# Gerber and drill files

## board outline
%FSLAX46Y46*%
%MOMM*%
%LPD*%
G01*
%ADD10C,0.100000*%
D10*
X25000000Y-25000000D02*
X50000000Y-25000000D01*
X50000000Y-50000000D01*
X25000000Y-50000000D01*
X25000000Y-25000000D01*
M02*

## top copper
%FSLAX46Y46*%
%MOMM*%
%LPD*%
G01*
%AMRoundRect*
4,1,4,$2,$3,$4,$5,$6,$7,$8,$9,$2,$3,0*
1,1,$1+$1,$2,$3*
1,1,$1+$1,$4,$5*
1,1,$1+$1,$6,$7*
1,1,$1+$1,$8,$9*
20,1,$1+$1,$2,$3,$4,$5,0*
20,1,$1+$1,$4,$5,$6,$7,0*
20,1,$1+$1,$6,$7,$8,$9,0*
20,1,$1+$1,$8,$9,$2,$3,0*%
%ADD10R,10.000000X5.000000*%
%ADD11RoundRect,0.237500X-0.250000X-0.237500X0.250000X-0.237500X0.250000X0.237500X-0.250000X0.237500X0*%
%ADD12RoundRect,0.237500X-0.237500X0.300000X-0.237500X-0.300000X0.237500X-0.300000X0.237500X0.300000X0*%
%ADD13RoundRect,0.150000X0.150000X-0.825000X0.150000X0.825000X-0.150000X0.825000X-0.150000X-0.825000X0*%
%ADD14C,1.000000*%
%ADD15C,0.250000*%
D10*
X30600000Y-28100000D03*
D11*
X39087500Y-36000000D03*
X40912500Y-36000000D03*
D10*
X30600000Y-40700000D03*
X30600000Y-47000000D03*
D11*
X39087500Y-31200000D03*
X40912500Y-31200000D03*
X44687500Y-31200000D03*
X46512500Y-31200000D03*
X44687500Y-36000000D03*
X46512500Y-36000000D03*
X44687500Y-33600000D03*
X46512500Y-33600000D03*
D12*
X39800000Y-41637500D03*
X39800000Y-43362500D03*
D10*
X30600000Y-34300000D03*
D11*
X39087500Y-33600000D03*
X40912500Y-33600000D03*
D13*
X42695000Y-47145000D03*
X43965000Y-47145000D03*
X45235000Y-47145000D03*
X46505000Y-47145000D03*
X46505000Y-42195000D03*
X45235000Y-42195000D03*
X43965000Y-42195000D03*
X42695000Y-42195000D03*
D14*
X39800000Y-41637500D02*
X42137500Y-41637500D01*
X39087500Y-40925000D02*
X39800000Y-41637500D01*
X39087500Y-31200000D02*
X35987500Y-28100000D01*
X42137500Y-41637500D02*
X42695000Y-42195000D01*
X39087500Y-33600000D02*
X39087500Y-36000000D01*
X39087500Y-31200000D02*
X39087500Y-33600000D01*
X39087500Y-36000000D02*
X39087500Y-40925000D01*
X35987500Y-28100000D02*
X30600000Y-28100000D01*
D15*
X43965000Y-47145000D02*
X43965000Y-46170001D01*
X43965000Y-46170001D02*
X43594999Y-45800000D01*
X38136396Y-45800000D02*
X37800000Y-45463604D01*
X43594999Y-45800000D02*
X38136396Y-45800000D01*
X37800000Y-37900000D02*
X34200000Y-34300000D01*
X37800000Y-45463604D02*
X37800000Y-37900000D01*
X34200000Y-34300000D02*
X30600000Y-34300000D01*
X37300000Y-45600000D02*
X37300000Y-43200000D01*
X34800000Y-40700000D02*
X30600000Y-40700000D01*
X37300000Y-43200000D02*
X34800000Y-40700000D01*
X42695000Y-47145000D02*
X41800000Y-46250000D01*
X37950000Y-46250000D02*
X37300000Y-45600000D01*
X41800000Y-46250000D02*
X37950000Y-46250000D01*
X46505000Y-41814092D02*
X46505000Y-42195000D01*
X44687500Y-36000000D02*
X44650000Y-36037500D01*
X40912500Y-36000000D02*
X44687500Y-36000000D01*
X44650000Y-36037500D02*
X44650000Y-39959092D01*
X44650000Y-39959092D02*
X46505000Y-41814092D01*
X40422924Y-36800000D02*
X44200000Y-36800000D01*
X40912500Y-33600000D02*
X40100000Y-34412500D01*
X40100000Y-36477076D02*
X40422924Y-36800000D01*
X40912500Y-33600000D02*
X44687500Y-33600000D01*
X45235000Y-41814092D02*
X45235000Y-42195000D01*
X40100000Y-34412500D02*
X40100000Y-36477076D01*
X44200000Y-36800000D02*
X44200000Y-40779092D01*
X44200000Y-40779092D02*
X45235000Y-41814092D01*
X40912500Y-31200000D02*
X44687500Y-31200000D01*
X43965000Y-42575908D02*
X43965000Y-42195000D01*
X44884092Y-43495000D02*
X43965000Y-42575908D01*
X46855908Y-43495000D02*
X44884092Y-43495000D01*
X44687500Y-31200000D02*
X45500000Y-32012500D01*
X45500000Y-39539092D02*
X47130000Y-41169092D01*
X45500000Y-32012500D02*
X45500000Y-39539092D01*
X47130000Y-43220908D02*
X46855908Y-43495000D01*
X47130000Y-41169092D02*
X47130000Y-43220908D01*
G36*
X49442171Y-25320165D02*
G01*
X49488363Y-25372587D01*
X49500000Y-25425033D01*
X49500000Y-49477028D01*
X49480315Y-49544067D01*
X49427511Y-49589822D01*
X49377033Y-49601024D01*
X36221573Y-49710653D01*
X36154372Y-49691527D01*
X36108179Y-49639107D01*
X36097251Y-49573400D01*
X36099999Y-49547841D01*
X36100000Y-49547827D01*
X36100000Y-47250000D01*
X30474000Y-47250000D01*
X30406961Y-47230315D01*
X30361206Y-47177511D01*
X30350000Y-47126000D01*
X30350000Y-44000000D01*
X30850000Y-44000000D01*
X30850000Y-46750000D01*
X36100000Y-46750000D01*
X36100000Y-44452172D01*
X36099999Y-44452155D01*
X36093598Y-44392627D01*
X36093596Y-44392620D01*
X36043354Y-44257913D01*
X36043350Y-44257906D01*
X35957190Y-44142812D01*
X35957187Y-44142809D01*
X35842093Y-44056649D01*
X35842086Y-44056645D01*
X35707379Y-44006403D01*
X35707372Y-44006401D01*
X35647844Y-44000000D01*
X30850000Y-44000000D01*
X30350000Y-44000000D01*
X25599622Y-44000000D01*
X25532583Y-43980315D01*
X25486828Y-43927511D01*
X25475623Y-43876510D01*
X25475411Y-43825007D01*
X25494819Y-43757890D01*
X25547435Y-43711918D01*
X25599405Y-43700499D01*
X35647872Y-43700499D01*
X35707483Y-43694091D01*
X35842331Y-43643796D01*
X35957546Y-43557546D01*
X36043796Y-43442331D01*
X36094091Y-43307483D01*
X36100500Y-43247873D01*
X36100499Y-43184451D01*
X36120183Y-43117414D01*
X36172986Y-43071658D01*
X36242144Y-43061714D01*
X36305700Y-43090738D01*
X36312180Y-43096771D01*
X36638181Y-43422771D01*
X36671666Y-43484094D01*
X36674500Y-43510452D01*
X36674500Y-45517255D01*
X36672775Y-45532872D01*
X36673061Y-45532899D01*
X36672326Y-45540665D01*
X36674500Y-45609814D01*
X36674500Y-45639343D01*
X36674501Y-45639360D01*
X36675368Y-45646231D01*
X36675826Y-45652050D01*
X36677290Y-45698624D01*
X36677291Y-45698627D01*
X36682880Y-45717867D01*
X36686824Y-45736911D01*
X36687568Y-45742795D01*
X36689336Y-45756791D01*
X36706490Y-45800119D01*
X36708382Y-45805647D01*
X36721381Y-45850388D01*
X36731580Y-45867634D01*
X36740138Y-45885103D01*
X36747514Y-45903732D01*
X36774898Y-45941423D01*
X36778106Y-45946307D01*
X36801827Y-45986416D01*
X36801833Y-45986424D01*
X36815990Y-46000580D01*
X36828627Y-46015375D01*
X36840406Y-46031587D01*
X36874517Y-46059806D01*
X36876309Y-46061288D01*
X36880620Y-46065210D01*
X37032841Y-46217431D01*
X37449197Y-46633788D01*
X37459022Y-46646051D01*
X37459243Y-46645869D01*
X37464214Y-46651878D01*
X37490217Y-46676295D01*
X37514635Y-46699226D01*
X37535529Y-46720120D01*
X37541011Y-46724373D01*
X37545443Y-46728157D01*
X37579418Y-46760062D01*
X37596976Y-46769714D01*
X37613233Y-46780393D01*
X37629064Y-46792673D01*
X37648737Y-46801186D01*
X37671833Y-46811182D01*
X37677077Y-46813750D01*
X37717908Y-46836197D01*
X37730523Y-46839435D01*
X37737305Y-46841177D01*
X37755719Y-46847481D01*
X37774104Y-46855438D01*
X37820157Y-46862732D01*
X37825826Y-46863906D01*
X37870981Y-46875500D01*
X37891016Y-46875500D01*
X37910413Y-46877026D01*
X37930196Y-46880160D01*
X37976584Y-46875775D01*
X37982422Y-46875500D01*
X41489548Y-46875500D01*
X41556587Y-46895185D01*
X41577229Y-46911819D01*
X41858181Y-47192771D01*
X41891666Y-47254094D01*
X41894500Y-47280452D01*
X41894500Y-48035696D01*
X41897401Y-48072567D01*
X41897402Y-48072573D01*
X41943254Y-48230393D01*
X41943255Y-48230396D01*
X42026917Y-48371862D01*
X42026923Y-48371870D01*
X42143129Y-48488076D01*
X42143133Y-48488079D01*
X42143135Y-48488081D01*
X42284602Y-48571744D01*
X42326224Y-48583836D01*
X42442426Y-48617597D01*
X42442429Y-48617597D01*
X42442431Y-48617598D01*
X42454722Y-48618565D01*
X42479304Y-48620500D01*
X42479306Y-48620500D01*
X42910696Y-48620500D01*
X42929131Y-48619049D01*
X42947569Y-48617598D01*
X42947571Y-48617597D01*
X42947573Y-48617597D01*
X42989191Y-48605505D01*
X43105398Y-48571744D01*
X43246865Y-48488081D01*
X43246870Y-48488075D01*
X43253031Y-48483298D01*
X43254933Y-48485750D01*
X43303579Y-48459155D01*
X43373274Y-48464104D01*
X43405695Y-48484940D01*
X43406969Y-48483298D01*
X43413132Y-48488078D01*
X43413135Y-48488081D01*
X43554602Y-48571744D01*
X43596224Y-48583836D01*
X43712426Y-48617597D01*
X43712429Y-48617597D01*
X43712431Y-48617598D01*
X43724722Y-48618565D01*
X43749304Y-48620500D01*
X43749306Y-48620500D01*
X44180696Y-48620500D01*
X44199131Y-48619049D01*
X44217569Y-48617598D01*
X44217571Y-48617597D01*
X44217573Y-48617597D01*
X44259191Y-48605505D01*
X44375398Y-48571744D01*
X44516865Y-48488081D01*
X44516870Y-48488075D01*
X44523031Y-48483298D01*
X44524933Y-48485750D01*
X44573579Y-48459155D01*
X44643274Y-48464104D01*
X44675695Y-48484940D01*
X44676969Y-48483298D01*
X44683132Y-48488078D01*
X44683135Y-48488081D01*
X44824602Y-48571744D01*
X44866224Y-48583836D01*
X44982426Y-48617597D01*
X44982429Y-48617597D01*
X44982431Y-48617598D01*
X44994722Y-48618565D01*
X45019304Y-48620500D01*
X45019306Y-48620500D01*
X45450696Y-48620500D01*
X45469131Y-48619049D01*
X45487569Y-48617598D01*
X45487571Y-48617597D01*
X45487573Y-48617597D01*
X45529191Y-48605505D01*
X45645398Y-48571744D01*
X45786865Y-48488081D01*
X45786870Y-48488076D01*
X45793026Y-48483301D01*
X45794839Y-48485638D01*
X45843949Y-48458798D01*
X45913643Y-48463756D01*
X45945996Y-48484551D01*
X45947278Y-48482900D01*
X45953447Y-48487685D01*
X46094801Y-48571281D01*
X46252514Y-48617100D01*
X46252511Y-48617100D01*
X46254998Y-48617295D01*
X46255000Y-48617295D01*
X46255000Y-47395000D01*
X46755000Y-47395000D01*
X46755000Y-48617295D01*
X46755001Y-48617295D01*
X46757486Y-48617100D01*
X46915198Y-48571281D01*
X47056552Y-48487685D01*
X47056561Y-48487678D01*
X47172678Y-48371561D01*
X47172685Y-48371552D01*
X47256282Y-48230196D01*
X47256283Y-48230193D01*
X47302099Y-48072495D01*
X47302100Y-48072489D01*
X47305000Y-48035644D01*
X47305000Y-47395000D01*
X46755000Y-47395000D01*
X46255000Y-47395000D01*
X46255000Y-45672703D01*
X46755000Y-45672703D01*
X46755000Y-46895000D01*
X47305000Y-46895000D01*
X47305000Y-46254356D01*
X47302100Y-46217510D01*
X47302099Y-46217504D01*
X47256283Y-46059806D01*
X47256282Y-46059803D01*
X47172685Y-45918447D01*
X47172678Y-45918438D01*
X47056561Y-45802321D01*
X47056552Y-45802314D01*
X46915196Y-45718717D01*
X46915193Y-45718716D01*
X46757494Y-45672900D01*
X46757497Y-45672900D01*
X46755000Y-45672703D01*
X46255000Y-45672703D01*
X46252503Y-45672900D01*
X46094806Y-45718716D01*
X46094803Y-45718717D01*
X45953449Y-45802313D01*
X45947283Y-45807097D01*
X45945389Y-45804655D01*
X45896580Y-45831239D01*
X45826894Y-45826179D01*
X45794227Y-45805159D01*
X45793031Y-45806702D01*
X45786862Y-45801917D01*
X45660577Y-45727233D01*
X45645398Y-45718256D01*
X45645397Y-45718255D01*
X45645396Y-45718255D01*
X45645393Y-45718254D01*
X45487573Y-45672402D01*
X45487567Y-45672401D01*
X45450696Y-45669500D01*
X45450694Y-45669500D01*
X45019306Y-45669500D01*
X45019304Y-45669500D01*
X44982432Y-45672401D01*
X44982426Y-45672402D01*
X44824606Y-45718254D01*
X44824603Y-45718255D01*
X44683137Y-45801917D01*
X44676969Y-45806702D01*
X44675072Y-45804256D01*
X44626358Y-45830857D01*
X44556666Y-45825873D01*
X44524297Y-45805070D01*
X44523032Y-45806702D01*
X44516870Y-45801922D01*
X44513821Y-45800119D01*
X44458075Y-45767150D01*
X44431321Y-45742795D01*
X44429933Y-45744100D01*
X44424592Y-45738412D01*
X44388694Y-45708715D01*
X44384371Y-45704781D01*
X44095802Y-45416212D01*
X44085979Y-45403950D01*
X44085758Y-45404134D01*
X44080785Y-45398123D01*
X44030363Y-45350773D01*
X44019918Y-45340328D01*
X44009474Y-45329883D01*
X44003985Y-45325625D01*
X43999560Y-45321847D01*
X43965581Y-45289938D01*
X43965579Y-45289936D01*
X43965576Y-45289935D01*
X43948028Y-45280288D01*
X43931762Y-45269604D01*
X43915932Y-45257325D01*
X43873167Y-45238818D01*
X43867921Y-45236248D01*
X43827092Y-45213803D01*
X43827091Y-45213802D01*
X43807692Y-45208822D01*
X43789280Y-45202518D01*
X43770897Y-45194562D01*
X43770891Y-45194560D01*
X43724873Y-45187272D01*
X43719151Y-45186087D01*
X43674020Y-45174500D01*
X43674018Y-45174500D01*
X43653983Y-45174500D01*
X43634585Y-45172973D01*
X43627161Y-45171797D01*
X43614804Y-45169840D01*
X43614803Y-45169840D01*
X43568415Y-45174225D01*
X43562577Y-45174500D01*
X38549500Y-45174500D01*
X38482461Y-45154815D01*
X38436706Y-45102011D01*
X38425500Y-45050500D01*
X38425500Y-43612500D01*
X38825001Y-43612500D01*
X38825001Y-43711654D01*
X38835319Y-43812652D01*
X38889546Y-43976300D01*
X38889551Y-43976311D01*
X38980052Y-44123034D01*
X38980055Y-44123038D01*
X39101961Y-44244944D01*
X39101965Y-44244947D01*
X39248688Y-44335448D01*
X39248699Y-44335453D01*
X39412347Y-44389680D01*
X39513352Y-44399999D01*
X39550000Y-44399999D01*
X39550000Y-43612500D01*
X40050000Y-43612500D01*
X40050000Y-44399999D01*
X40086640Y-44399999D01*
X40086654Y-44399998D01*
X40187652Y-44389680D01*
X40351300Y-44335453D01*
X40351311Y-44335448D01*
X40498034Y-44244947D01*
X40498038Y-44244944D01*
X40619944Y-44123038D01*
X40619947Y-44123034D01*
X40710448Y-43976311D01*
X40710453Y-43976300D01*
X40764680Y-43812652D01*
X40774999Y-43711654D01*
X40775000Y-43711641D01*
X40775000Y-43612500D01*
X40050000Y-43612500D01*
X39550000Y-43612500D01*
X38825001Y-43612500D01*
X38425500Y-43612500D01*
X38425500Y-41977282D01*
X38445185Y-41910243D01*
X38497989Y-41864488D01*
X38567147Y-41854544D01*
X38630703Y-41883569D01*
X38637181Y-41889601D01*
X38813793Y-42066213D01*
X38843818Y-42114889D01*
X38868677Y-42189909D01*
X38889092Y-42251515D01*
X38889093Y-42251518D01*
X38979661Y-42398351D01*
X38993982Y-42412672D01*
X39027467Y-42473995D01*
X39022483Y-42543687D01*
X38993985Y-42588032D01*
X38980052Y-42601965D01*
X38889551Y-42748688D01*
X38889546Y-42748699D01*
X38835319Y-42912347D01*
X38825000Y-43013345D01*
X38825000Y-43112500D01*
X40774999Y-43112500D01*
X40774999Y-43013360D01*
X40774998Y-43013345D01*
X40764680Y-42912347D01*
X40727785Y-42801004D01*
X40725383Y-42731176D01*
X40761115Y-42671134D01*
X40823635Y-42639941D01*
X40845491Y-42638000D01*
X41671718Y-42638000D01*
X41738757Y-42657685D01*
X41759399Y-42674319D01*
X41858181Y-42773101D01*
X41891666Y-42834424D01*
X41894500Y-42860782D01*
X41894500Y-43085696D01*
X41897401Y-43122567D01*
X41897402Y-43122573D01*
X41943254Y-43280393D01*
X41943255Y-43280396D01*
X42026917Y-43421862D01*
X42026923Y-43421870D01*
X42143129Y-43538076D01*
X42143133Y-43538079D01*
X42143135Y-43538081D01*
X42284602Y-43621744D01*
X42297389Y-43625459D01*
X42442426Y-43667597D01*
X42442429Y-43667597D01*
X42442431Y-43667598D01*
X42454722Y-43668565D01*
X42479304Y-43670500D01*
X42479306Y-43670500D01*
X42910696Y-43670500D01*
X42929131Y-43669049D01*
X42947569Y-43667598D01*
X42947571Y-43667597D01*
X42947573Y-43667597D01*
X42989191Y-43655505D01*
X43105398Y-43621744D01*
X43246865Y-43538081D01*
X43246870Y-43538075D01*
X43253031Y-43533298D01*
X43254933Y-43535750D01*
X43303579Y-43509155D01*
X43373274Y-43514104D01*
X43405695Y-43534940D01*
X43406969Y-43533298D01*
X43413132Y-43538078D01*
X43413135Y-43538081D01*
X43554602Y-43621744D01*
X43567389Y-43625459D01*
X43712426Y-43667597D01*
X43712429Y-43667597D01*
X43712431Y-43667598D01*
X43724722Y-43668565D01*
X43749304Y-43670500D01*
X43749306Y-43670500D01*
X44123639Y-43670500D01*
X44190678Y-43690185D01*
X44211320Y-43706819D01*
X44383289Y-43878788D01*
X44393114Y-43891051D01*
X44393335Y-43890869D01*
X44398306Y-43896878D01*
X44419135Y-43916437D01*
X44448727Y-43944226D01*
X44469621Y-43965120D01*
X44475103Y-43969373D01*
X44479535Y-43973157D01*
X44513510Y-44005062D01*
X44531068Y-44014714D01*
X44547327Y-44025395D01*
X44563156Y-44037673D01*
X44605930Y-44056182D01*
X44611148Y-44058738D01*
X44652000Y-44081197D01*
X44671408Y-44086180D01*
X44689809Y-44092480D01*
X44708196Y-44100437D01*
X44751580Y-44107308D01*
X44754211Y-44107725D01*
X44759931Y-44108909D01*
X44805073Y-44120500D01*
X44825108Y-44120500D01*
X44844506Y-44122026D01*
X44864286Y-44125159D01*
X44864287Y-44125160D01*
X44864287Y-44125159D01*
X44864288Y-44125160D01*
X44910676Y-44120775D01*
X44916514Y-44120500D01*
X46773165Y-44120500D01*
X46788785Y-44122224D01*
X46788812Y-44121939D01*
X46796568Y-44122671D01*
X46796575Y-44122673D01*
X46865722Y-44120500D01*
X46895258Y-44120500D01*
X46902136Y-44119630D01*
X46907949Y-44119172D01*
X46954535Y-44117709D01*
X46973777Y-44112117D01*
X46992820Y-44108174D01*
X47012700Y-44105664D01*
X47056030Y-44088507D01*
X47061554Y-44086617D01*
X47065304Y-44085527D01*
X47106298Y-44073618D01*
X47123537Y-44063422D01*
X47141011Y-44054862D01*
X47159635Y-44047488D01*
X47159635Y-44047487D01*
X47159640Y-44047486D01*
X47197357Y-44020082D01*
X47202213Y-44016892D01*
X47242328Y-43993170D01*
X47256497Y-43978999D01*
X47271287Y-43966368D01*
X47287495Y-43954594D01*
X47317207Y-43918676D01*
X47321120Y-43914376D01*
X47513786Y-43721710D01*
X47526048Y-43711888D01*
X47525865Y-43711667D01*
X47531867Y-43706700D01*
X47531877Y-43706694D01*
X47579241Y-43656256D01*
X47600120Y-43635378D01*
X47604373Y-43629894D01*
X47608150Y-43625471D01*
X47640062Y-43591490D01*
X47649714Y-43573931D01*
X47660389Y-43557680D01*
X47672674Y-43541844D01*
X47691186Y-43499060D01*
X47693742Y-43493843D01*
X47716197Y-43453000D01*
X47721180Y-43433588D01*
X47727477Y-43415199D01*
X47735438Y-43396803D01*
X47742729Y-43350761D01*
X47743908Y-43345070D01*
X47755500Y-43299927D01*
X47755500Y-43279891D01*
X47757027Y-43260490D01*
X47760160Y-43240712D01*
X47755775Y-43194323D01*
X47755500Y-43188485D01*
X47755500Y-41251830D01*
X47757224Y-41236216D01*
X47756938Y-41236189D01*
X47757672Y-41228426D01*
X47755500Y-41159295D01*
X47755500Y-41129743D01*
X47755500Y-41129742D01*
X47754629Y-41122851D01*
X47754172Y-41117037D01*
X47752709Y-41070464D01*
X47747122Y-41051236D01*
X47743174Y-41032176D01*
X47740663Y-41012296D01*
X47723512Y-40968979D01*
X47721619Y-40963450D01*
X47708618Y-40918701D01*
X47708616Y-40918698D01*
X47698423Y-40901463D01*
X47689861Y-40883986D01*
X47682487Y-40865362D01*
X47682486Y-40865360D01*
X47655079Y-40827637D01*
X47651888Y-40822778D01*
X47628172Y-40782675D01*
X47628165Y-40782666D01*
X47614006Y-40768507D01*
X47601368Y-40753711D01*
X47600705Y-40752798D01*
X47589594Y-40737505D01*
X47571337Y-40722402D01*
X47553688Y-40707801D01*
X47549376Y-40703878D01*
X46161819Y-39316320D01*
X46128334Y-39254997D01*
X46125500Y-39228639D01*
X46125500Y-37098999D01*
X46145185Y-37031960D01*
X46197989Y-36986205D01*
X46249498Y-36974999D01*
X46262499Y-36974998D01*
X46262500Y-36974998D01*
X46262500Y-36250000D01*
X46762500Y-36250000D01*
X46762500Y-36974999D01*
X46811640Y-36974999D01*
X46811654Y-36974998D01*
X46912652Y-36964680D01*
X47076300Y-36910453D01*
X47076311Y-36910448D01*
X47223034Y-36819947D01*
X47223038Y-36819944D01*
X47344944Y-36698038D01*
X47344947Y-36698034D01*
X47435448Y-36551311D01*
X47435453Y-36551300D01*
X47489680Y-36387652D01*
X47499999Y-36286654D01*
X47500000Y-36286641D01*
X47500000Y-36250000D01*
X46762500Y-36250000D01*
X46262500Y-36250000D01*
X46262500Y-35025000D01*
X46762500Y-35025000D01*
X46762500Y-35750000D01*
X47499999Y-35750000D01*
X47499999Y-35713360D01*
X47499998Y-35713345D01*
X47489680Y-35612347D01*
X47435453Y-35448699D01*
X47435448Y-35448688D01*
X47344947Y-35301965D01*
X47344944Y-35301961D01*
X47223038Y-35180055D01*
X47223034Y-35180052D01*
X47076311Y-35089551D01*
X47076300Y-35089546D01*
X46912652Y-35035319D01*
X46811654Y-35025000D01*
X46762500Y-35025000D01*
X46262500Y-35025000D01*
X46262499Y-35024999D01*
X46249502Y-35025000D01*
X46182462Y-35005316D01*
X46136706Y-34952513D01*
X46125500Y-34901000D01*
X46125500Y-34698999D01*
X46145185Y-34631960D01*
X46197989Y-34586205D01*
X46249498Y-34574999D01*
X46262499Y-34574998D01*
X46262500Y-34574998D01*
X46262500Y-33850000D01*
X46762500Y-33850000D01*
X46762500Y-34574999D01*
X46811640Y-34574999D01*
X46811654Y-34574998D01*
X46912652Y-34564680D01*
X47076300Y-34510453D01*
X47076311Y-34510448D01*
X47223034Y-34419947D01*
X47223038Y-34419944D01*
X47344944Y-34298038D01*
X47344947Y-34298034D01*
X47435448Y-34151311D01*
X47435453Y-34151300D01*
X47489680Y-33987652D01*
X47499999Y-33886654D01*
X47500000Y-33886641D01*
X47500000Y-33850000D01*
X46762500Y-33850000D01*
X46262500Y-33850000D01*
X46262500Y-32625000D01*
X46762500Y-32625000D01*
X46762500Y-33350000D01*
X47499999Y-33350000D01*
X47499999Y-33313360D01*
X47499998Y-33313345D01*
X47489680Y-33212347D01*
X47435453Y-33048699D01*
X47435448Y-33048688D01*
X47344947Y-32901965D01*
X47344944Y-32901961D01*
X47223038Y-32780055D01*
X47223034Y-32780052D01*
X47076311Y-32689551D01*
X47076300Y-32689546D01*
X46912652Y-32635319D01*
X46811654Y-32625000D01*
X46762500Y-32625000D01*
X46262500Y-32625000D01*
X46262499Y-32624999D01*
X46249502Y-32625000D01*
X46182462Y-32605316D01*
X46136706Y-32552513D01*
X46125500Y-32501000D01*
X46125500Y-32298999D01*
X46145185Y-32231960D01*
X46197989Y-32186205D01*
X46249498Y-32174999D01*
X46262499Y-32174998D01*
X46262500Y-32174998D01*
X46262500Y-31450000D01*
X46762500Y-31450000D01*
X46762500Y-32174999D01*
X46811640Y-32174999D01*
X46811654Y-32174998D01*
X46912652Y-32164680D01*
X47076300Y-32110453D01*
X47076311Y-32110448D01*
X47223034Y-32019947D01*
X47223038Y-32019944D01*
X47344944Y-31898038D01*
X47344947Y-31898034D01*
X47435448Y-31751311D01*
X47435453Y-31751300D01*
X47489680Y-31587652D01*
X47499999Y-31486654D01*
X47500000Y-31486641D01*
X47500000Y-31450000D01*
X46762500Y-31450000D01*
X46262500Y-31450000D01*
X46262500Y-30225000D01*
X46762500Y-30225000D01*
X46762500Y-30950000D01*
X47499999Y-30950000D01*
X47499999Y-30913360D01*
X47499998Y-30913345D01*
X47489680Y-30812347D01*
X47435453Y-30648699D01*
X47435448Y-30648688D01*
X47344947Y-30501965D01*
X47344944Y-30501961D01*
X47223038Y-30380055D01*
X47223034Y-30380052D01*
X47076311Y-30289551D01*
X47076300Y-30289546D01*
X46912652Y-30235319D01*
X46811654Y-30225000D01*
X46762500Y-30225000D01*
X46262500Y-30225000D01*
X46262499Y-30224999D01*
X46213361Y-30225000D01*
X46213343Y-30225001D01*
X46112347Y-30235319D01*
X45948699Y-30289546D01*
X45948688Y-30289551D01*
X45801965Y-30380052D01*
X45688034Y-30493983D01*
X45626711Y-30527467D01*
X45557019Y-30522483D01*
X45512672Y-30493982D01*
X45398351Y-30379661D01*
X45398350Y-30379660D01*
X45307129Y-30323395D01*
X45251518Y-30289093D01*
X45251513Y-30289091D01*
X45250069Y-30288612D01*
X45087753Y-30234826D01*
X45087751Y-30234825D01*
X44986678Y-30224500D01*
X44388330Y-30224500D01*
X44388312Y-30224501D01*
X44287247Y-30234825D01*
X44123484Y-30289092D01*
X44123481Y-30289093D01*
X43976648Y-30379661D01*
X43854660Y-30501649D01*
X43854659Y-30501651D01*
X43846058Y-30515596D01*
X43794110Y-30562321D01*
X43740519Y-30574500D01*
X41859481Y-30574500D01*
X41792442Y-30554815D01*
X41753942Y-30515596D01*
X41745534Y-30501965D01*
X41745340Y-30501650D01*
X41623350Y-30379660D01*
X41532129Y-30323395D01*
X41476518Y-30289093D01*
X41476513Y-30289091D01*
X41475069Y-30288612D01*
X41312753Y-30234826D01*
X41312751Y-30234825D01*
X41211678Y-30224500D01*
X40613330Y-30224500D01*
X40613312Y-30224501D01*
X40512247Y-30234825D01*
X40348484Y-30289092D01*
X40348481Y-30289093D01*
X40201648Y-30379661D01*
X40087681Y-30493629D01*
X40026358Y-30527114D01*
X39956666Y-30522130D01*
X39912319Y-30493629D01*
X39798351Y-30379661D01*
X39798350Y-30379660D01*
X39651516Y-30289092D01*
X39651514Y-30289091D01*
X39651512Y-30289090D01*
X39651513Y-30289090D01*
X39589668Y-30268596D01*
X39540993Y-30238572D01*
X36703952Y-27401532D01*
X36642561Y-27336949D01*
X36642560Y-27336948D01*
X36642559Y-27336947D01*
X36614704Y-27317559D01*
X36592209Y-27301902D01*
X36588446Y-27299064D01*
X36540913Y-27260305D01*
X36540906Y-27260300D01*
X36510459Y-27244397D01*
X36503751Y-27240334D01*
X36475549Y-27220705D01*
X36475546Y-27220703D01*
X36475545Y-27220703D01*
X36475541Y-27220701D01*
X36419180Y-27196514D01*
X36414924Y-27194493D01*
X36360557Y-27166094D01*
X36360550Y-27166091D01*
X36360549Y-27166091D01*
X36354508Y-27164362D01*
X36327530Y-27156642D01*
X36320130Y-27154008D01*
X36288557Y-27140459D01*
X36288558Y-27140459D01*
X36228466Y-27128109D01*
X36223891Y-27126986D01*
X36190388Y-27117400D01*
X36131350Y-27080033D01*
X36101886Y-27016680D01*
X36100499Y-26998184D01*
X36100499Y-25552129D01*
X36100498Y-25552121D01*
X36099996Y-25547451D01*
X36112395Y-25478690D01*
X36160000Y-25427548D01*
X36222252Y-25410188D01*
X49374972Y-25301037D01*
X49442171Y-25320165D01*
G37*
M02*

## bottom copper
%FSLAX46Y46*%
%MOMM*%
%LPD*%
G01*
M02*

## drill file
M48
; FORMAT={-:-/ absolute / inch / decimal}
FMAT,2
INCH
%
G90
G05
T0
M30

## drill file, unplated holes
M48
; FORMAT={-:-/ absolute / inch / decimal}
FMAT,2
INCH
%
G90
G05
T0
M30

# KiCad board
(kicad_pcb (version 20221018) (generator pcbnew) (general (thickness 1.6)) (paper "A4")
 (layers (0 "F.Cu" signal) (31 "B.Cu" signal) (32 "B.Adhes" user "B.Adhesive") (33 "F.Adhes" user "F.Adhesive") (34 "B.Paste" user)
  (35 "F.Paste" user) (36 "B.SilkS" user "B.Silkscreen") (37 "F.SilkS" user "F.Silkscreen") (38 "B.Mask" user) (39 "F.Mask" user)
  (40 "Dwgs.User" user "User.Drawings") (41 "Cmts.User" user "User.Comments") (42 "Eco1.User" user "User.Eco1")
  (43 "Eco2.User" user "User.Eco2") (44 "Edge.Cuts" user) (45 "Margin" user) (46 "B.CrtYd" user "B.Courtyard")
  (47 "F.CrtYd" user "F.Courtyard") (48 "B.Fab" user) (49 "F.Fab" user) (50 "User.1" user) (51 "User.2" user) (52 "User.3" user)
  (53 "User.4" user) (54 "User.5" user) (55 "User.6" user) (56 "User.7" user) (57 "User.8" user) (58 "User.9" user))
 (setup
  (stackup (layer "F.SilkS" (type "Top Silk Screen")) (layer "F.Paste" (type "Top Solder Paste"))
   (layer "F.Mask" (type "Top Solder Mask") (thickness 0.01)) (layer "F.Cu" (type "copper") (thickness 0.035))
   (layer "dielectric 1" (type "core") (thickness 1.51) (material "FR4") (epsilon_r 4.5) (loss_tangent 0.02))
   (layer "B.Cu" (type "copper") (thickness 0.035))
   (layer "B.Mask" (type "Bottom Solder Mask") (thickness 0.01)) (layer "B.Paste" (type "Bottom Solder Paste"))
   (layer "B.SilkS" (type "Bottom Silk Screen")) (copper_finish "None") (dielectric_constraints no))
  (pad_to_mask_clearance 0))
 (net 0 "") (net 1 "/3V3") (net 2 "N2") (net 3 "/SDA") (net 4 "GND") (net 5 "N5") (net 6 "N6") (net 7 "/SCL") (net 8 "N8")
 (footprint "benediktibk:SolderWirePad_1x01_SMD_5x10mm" (layer "F.Cu") (at 30.6 28.1 -90)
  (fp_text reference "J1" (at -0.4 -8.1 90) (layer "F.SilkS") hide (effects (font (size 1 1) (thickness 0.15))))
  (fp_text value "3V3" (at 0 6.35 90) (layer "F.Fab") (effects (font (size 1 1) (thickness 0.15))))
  (pad "1" smd rect (at 0 0 270) (size 5 10) (layers "F.Cu" "F.Paste" "F.Mask") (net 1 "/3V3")))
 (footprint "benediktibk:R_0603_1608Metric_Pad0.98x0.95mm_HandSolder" (layer "F.Cu") (at 40 36)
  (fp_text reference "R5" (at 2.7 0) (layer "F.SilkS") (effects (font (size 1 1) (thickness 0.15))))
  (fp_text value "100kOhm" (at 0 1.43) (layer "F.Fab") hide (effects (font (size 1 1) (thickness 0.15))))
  (pad "1" smd roundrect (at -0.9125 0) (size 0.975 0.95) (layers "F.Cu" "F.Paste" "F.Mask") (roundrect_rratio 0.25) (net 1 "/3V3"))
  (pad "2" smd roundrect (at 0.9125 0) (size 0.975 0.95) (layers "F.Cu" "F.Paste" "F.Mask") (roundrect_rratio 0.25) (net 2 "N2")))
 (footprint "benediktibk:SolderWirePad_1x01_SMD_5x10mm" (layer "F.Cu") (at 30.6 40.7 -90)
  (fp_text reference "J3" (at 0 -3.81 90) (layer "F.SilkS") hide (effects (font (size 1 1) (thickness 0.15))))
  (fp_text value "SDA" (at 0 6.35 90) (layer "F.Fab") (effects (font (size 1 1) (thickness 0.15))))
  (pad "1" smd rect (at 0 0 270) (size 5 10) (layers "F.Cu" "F.Paste" "F.Mask") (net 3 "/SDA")))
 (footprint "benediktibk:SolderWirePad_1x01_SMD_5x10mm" (layer "F.Cu") (at 30.6 47 -90)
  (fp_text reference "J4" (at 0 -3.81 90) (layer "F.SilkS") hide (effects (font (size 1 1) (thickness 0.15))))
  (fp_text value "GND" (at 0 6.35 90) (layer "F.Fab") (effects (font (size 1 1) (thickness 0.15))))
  (pad "1" smd rect (at 0 0 270) (size 5 10) (layers "F.Cu" "F.Paste" "F.Mask") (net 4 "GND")))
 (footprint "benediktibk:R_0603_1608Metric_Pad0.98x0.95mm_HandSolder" (layer "F.Cu") (at 40 31.2)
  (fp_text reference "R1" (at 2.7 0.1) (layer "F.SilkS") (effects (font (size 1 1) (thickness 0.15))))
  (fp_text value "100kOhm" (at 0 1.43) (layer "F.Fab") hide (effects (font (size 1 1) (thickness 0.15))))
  (pad "1" smd roundrect (at -0.9125 0) (size 0.975 0.95) (layers "F.Cu" "F.Paste" "F.Mask") (roundrect_rratio 0.25) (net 1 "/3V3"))
  (pad "2" smd roundrect (at 0.9125 0) (size 0.975 0.95) (layers "F.Cu" "F.Paste" "F.Mask") (roundrect_rratio 0.25) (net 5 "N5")))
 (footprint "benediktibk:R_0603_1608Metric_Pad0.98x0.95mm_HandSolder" (layer "F.Cu") (at 45.6 31.2)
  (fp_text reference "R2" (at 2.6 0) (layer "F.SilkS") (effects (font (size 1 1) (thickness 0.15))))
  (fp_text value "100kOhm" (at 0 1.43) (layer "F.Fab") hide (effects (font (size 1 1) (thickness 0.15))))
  (pad "1" smd roundrect (at -0.9125 0) (size 0.975 0.95) (layers "F.Cu" "F.Paste" "F.Mask") (roundrect_rratio 0.25) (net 5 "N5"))
  (pad "2" smd roundrect (at 0.9125 0) (size 0.975 0.95) (layers "F.Cu" "F.Paste" "F.Mask") (roundrect_rratio 0.25) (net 4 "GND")))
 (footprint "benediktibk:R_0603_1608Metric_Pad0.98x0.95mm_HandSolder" (layer "F.Cu") (at 45.6 36)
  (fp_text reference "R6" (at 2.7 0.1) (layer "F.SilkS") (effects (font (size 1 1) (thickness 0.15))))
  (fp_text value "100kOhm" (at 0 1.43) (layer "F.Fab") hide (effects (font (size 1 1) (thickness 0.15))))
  (pad "1" smd roundrect (at -0.9125 0) (size 0.975 0.95) (layers "F.Cu" "F.Paste" "F.Mask") (roundrect_rratio 0.25) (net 2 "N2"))
  (pad "2" smd roundrect (at 0.9125 0) (size 0.975 0.95) (layers "F.Cu" "F.Paste" "F.Mask") (roundrect_rratio 0.25) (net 4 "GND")))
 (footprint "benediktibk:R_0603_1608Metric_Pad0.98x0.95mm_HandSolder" (layer "F.Cu") (at 45.6 33.6)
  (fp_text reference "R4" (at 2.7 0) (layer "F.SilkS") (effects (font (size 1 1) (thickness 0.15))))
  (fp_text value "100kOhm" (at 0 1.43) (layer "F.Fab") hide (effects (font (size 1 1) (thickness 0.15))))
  (pad "1" smd roundrect (at -0.9125 0) (size 0.975 0.95) (layers "F.Cu" "F.Paste" "F.Mask") (roundrect_rratio 0.25) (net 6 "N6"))
  (pad "2" smd roundrect (at 0.9125 0) (size 0.975 0.95) (layers "F.Cu" "F.Paste" "F.Mask") (roundrect_rratio 0.25) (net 4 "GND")))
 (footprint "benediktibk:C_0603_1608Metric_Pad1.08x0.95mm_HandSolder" (layer "F.Cu") (at 39.8 42.5 -90)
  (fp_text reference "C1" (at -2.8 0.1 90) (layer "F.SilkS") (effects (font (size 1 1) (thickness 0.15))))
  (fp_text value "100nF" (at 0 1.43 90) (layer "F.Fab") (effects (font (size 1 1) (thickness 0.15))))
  (pad "1" smd roundrect (at -0.8625 0 270) (size 1.075 0.95) (layers "F.Cu" "F.Paste" "F.Mask") (roundrect_rratio 0.25) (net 1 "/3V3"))
  (pad "2" smd roundrect (at 0.8625 0 270) (size 1.075 0.95) (layers "F.Cu" "F.Paste" "F.Mask") (roundrect_rratio 0.25) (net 4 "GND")))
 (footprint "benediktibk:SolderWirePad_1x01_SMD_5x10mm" (layer "F.Cu") (at 30.6 34.3 -90)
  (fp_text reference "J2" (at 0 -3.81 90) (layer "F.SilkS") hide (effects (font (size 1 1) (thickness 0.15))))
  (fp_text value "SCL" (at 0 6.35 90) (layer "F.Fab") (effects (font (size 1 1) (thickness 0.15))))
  (pad "1" smd rect (at 0 0 270) (size 5 10) (layers "F.Cu" "F.Paste" "F.Mask") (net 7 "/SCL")))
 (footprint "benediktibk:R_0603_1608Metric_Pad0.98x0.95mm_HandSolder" (layer "F.Cu") (at 40 33.6)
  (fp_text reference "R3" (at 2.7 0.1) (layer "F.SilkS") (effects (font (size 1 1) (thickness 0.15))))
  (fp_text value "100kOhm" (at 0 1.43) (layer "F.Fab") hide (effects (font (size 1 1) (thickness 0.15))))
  (pad "1" smd roundrect (at -0.9125 0) (size 0.975 0.95) (layers "F.Cu" "F.Paste" "F.Mask") (roundrect_rratio 0.25) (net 1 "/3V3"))
  (pad "2" smd roundrect (at 0.9125 0) (size 0.975 0.95) (layers "F.Cu" "F.Paste" "F.Mask") (roundrect_rratio 0.25) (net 6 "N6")))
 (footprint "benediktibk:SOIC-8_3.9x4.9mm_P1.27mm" (layer "F.Cu") (at 44.6 44.67 90)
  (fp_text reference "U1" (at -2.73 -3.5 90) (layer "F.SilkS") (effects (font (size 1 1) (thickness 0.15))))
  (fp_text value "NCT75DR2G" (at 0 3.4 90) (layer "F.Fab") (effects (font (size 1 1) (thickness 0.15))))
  (pad "1" smd roundrect (at -2.475 -1.905 90) (size 1.95 0.6) (layers "F.Cu" "F.Paste" "F.Mask") (roundrect_rratio 0.25) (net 3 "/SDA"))
  (pad "2" smd roundrect (at -2.475 -0.635 90) (size 1.95 0.6) (layers "F.Cu" "F.Paste" "F.Mask") (roundrect_rratio 0.25) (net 7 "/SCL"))
  (pad "3" smd roundrect (at -2.475 0.635 90) (size 1.95 0.6) (layers "F.Cu" "F.Paste" "F.Mask") (roundrect_rratio 0.25) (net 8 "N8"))
  (pad "4" smd roundrect (at -2.475 1.905 90) (size 1.95 0.6) (layers "F.Cu" "F.Paste" "F.Mask") (roundrect_rratio 0.25) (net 4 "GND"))
  (pad "5" smd roundrect (at 2.475 1.905 90) (size 1.95 0.6) (layers "F.Cu" "F.Paste" "F.Mask") (roundrect_rratio 0.25) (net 2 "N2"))
  (pad "6" smd roundrect (at 2.475 0.635 90) (size 1.95 0.6) (layers "F.Cu" "F.Paste" "F.Mask") (roundrect_rratio 0.25) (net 6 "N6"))
  (pad "7" smd roundrect (at 2.475 -0.635 90) (size 1.95 0.6) (layers "F.Cu" "F.Paste" "F.Mask") (roundrect_rratio 0.25) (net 5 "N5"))
  (pad "8" smd roundrect (at 2.475 -1.905 90) (size 1.95 0.6) (layers "F.Cu" "F.Paste" "F.Mask") (roundrect_rratio 0.25) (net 1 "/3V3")))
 (gr_rect (start 25 25) (end 50 50) (stroke (width 0.1) (type default)) (fill none) (layer "Edge.Cuts"))
 (segment (start 39.8 41.6375) (end 42.1375 41.6375) (width 1) (layer "F.Cu") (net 1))
 (segment (start 39.0875 40.925) (end 39.8 41.6375) (width 1) (layer "F.Cu") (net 1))
 (segment (start 39.0875 31.2) (end 35.9875 28.1) (width 1) (layer "F.Cu") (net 1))
 (segment (start 42.1375 41.6375) (end 42.695 42.195) (width 1) (layer "F.Cu") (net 1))
 (segment (start 39.0875 33.6) (end 39.0875 36) (width 1) (layer "F.Cu") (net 1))
 (segment (start 39.0875 31.2) (end 39.0875 33.6) (width 1) (layer "F.Cu") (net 1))
 (segment (start 39.0875 36) (end 39.0875 40.925) (width 1) (layer "F.Cu") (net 1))
 (segment (start 35.9875 28.1) (end 30.6 28.1) (width 1) (layer "F.Cu") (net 1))
 (segment (start 43.965 47.145) (end 43.965 46.170001) (width 0.25) (layer "F.Cu") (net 7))
 (segment (start 43.965 46.170001) (end 43.594999 45.8) (width 0.25) (layer "F.Cu") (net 7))
 (segment (start 38.136396 45.8) (end 37.8 45.463604) (width 0.25) (layer "F.Cu") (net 7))
 (segment (start 43.594999 45.8) (end 38.136396 45.8) (width 0.25) (layer "F.Cu") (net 7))
 (segment (start 37.8 37.9) (end 34.2 34.3) (width 0.25) (layer "F.Cu") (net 7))
 (segment (start 37.8 45.463604) (end 37.8 37.9) (width 0.25) (layer "F.Cu") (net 7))
 (segment (start 34.2 34.3) (end 30.6 34.3) (width 0.25) (layer "F.Cu") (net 7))
 (segment (start 37.3 45.6) (end 37.3 43.2) (width 0.25) (layer "F.Cu") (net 3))
 (segment (start 34.8 40.7) (end 30.6 40.7) (width 0.25) (layer "F.Cu") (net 3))
 (segment (start 37.3 43.2) (end 34.8 40.7) (width 0.25) (layer "F.Cu") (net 3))
 (segment (start 42.695 47.145) (end 41.8 46.25) (width 0.25) (layer "F.Cu") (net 3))
 (segment (start 37.95 46.25) (end 37.3 45.6) (width 0.25) (layer "F.Cu") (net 3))
 (segment (start 41.8 46.25) (end 37.95 46.25) (width 0.25) (layer "F.Cu") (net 3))
 (segment (start 46.505 41.814092) (end 46.505 42.195) (width 0.25) (layer "F.Cu") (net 2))
 (segment (start 44.6875 36) (end 44.65 36.0375) (width 0.25) (layer "F.Cu") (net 2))
 (segment (start 40.9125 36) (end 44.6875 36) (width 0.25) (layer "F.Cu") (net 2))
 (segment (start 44.65 36.0375) (end 44.65 39.959092) (width 0.25) (layer "F.Cu") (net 2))
 (segment (start 44.65 39.959092) (end 46.505 41.814092) (width 0.25) (layer "F.Cu") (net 2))
 (segment (start 40.422924 36.8) (end 44.2 36.8) (width 0.25) (layer "F.Cu") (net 6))
 (segment (start 40.9125 33.6) (end 40.1 34.4125) (width 0.25) (layer "F.Cu") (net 6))
 (segment (start 40.1 36.477076) (end 40.422924 36.8) (width 0.25) (layer "F.Cu") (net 6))
 (segment (start 40.9125 33.6) (end 44.6875 33.6) (width 0.25) (layer "F.Cu") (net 6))
 (segment (start 45.235 41.814092) (end 45.235 42.195) (width 0.25) (layer "F.Cu") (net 6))
 (segment (start 40.1 34.4125) (end 40.1 36.477076) (width 0.25) (layer "F.Cu") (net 6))
 (segment (start 44.2 36.8) (end 44.2 40.779092) (width 0.25) (layer "F.Cu") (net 6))
 (segment (start 44.2 40.779092) (end 45.235 41.814092) (width 0.25) (layer "F.Cu") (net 6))
 (segment (start 40.9125 31.2) (end 44.6875 31.2) (width 0.25) (layer "F.Cu") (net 5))
 (segment (start 43.965 42.575908) (end 43.965 42.195) (width 0.25) (layer "F.Cu") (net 5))
 (segment (start 44.884092 43.495) (end 43.965 42.575908) (width 0.25) (layer "F.Cu") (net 5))
 (segment (start 46.855908 43.495) (end 44.884092 43.495) (width 0.25) (layer "F.Cu") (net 5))
 (segment (start 44.6875 31.2) (end 45.5 32.0125) (width 0.25) (layer "F.Cu") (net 5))
 (segment (start 45.5 39.539092) (end 47.13 41.169092) (width 0.25) (layer "F.Cu") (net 5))
 (segment (start 45.5 32.0125) (end 45.5 39.539092) (width 0.25) (layer "F.Cu") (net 5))
 (segment (start 47.13 43.220908) (end 46.855908 43.495) (width 0.25) (layer "F.Cu") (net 5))
 (segment (start 47.13 41.169092) (end 47.13 43.220908) (width 0.25) (layer "F.Cu") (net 5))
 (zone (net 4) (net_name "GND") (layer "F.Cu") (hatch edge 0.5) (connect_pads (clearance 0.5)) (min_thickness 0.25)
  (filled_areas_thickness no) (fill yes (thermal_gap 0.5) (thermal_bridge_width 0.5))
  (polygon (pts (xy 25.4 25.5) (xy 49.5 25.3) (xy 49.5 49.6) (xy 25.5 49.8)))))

